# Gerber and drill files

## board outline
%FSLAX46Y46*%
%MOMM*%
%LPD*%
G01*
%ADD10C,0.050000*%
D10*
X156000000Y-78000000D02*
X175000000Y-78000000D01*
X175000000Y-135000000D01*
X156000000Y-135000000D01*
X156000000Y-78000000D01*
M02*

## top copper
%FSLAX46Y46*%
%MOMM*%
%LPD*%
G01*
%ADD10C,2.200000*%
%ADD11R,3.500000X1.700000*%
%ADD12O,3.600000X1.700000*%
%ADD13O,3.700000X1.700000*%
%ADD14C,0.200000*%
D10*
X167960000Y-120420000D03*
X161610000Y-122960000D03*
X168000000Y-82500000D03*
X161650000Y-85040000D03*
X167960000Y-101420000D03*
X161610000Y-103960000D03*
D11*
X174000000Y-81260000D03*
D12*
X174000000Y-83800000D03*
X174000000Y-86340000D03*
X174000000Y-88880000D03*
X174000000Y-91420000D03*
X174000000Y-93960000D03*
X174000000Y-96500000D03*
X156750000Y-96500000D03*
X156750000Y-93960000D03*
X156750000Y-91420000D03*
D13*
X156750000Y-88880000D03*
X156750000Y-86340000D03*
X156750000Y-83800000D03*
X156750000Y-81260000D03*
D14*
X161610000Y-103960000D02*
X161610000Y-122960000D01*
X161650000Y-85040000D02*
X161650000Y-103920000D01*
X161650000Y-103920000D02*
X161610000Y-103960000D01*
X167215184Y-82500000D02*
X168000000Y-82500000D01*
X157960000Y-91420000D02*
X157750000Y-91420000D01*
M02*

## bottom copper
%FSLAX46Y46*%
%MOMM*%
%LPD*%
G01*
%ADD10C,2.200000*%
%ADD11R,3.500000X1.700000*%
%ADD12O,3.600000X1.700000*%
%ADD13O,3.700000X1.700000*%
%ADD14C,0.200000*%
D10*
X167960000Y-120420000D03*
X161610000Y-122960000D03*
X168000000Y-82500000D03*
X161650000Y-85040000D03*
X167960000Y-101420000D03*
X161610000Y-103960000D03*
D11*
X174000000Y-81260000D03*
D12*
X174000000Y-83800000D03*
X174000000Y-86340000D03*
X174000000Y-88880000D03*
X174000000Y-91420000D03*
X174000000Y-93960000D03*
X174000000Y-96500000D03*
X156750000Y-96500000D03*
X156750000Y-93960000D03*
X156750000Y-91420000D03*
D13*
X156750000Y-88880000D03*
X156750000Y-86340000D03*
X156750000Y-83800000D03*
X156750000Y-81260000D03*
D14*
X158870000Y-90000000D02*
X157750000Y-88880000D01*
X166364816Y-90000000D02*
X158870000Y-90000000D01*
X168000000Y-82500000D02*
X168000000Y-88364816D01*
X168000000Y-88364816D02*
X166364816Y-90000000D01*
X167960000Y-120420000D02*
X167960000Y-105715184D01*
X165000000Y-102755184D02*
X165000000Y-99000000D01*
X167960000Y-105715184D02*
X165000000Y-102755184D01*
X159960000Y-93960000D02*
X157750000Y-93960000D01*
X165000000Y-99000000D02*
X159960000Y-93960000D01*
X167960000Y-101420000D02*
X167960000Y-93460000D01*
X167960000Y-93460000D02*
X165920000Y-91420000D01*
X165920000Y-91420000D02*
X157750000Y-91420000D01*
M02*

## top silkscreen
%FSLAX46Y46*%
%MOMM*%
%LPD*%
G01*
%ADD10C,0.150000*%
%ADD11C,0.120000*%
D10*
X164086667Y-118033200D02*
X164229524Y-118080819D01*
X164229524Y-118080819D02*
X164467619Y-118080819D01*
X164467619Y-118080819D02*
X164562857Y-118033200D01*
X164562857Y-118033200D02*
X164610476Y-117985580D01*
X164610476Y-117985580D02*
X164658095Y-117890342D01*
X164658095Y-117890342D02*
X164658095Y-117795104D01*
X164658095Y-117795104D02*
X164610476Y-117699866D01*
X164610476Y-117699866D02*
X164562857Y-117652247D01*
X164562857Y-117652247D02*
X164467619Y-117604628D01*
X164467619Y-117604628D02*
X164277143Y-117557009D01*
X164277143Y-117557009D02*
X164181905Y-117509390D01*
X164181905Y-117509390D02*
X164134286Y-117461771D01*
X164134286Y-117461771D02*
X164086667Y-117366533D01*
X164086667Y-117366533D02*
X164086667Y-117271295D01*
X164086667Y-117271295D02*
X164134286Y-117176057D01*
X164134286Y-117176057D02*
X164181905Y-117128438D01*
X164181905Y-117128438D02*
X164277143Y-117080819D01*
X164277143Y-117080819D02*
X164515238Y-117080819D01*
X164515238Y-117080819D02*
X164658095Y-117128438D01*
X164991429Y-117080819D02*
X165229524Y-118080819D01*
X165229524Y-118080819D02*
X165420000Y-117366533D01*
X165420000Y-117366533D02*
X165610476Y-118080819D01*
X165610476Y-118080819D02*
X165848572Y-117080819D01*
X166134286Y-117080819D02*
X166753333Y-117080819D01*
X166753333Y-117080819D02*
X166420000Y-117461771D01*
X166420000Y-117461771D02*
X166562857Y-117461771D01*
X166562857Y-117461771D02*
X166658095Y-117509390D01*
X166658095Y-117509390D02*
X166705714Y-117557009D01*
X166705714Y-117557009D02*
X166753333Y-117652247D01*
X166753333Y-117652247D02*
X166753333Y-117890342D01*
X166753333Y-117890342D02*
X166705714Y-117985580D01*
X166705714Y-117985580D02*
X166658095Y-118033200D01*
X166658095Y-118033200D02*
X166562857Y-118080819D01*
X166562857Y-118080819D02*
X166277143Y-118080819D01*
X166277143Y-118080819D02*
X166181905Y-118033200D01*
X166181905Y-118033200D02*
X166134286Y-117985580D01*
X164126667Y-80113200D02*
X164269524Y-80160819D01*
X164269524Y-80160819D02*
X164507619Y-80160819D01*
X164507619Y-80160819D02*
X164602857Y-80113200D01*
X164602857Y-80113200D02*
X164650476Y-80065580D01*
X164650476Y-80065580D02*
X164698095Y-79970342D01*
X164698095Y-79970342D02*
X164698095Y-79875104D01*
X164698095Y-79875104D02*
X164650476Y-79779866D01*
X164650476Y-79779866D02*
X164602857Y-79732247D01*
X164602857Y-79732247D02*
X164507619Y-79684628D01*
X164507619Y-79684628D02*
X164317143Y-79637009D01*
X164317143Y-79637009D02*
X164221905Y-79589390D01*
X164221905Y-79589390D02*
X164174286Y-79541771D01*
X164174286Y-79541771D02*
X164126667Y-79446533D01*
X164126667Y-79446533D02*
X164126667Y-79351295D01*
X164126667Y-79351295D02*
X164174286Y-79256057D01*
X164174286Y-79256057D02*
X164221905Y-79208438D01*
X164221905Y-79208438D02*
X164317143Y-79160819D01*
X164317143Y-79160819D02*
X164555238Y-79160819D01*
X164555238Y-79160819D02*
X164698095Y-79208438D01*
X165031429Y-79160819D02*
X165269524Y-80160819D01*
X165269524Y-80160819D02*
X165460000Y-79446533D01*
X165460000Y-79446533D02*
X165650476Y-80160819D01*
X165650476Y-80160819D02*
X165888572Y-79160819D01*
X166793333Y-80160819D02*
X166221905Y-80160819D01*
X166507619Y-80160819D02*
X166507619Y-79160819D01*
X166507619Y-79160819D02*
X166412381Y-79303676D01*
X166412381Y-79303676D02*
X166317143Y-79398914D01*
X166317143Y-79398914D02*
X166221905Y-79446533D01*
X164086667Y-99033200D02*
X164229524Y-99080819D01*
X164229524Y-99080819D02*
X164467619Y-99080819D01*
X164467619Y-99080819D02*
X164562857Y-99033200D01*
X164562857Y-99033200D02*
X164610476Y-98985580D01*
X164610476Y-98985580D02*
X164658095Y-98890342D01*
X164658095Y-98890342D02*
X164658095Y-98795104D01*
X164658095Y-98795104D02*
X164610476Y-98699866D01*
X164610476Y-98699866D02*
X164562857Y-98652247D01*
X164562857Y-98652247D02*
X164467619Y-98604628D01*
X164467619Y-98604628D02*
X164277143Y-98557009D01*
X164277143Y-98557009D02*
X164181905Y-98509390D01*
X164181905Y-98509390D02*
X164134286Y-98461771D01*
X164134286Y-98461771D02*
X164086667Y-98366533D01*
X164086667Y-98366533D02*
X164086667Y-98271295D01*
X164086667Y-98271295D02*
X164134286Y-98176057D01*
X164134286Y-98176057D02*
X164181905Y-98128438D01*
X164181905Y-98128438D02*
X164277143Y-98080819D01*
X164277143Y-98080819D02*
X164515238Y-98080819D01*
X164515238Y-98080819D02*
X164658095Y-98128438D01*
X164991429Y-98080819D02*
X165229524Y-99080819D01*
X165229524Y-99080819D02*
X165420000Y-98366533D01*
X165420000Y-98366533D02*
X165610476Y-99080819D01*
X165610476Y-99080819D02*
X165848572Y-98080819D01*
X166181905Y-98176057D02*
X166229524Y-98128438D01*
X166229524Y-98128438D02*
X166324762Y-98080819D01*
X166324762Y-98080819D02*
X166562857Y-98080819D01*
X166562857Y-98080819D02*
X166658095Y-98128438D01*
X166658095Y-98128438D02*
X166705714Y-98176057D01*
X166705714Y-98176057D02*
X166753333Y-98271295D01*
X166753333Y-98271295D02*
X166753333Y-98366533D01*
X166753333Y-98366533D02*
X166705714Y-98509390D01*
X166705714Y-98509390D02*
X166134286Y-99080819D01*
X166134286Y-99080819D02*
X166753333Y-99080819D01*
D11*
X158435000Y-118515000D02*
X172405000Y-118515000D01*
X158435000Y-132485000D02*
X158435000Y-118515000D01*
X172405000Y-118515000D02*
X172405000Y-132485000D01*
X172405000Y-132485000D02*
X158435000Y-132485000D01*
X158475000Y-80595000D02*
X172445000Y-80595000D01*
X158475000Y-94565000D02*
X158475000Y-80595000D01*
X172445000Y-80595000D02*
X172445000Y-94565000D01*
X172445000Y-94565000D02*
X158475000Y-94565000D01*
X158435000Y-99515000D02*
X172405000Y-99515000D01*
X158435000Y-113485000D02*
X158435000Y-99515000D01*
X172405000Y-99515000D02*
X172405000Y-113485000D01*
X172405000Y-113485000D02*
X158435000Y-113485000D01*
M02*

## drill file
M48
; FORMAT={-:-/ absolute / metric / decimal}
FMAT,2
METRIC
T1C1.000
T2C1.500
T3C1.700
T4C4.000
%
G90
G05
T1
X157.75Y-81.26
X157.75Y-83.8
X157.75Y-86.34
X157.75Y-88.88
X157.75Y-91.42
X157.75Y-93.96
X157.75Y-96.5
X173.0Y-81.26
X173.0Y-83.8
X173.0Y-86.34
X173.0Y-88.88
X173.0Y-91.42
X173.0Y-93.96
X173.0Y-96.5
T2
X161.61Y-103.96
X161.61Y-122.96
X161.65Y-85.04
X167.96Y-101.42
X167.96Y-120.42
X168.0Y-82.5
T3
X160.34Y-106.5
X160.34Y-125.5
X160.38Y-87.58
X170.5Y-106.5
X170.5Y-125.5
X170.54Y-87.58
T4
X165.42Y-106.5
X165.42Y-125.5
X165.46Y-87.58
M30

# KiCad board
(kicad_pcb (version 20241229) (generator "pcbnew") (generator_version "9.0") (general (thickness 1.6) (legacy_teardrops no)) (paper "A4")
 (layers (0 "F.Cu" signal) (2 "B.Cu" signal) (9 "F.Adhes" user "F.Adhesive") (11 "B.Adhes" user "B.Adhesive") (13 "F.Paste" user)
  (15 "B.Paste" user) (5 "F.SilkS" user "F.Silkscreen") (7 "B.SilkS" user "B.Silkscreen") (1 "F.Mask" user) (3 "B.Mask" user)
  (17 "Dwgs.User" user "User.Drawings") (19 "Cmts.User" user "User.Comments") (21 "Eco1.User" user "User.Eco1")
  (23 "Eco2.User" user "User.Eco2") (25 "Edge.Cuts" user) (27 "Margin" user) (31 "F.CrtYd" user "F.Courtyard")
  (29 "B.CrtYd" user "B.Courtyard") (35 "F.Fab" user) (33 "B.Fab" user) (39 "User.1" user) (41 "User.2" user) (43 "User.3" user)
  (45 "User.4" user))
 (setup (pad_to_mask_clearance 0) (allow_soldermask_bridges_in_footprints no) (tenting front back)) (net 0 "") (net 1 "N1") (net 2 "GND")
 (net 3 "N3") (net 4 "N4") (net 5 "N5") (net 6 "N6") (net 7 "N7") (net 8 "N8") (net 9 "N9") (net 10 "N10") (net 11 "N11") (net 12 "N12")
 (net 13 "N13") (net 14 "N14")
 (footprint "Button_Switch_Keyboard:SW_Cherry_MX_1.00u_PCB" (layer "F.Cu") (at 167.96 120.42)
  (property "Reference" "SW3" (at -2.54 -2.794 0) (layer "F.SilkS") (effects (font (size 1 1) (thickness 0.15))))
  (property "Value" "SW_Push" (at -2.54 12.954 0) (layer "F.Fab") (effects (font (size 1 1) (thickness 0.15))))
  (fp_line (start -9.525 -1.905) (end 4.445 -1.905) (stroke (width 0.12) (type solid)) (layer "F.SilkS"))
  (fp_line (start -9.525 12.065) (end -9.525 -1.905) (stroke (width 0.12) (type solid)) (layer "F.SilkS"))
  (fp_line (start 4.445 -1.905) (end 4.445 12.065) (stroke (width 0.12) (type solid)) (layer "F.SilkS"))
  (fp_line (start 4.445 12.065) (end -9.525 12.065) (stroke (width 0.12) (type solid)) (layer "F.SilkS"))
  (pad "" np_thru_hole circle (at -7.62 5.08) (size 1.7 1.7) (drill 1.7) (layers "*.Cu" "*.Mask"))
  (pad "" np_thru_hole circle (at -2.54 5.08) (size 4 4) (drill 4) (layers "*.Cu" "*.Mask"))
  (pad "" np_thru_hole circle (at 2.54 5.08) (size 1.7 1.7) (drill 1.7) (layers "*.Cu" "*.Mask"))
  (pad "1" thru_hole circle (at 0 0) (size 2.2 2.2) (drill 1.5) (layers "*.Cu" "*.Mask") (remove_unused_layers no) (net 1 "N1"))
  (pad "2" thru_hole circle (at -6.35 2.54) (size 2.2 2.2) (drill 1.5) (layers "*.Cu" "*.Mask") (remove_unused_layers no) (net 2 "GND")))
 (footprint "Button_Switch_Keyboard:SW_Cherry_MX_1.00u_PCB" (layer "F.Cu") (at 168 82.5)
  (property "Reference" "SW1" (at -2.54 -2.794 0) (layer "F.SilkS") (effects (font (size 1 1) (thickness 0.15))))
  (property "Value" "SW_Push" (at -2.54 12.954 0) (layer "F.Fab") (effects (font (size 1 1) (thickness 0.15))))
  (fp_line (start -9.525 -1.905) (end 4.445 -1.905) (stroke (width 0.12) (type solid)) (layer "F.SilkS"))
  (fp_line (start -9.525 12.065) (end -9.525 -1.905) (stroke (width 0.12) (type solid)) (layer "F.SilkS"))
  (fp_line (start 4.445 -1.905) (end 4.445 12.065) (stroke (width 0.12) (type solid)) (layer "F.SilkS"))
  (fp_line (start 4.445 12.065) (end -9.525 12.065) (stroke (width 0.12) (type solid)) (layer "F.SilkS"))
  (pad "" np_thru_hole circle (at -7.62 5.08) (size 1.7 1.7) (drill 1.7) (layers "*.Cu" "*.Mask"))
  (pad "" np_thru_hole circle (at -2.54 5.08) (size 4 4) (drill 4) (layers "*.Cu" "*.Mask"))
  (pad "" np_thru_hole circle (at 2.54 5.08) (size 1.7 1.7) (drill 1.7) (layers "*.Cu" "*.Mask"))
  (pad "1" thru_hole circle (at 0 0) (size 2.2 2.2) (drill 1.5) (layers "*.Cu" "*.Mask") (remove_unused_layers no) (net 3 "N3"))
  (pad "2" thru_hole circle (at -6.35 2.54) (size 2.2 2.2) (drill 1.5) (layers "*.Cu" "*.Mask") (remove_unused_layers no) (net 2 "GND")))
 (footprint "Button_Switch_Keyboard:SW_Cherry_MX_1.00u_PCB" (layer "F.Cu") (at 167.96 101.42)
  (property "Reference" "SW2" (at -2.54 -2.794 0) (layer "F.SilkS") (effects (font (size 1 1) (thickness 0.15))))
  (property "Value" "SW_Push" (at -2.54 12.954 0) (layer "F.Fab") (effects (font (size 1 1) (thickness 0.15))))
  (fp_line (start -9.525 -1.905) (end 4.445 -1.905) (stroke (width 0.12) (type solid)) (layer "F.SilkS"))
  (fp_line (start -9.525 12.065) (end -9.525 -1.905) (stroke (width 0.12) (type solid)) (layer "F.SilkS"))
  (fp_line (start 4.445 -1.905) (end 4.445 12.065) (stroke (width 0.12) (type solid)) (layer "F.SilkS"))
  (fp_line (start 4.445 12.065) (end -9.525 12.065) (stroke (width 0.12) (type solid)) (layer "F.SilkS"))
  (pad "" np_thru_hole circle (at -7.62 5.08) (size 1.7 1.7) (drill 1.7) (layers "*.Cu" "*.Mask"))
  (pad "" np_thru_hole circle (at -2.54 5.08) (size 4 4) (drill 4) (layers "*.Cu" "*.Mask"))
  (pad "" np_thru_hole circle (at 2.54 5.08) (size 1.7 1.7) (drill 1.7) (layers "*.Cu" "*.Mask"))
  (pad "1" thru_hole circle (at 0 0) (size 2.2 2.2) (drill 1.5) (layers "*.Cu" "*.Mask") (remove_unused_layers no) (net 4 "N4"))
  (pad "2" thru_hole circle (at -6.35 2.54) (size 2.2 2.2) (drill 1.5) (layers "*.Cu" "*.Mask") (remove_unused_layers no) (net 2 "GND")))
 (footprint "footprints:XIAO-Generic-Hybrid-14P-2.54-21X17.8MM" (layer "B.Cu") (at 165.375 88.88 180)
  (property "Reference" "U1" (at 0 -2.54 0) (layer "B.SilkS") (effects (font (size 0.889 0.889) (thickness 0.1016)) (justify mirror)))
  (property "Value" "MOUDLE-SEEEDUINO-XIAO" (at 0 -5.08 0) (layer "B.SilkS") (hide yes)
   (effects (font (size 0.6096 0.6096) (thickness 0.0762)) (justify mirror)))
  (pad "1" thru_hole rect (at -7.625 7.62 180) (size 3.5 1.7) (drill 1 (offset -1 0)) (layers "*.Cu" "*.Mask") (remove_unused_layers no)
   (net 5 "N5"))
  (pad "2" thru_hole oval (at -7.625 5.08 180) (size 3.6 1.7) (drill 1 (offset -1 0)) (layers "*.Cu" "*.Mask") (remove_unused_layers no)
   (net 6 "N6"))
  (pad "3" thru_hole oval (at -7.625 2.54 180) (size 3.6 1.7) (drill 1 (offset -1 0)) (layers "*.Cu" "*.Mask") (remove_unused_layers no)
   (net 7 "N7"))
  (pad "4" thru_hole oval (at -7.625 0 180) (size 3.6 1.7) (drill 1 (offset -1 0)) (layers "*.Cu" "*.Mask") (remove_unused_layers no)
   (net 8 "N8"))
  (pad "5" thru_hole oval (at -7.625 -2.54 180) (size 3.6 1.7) (drill 1 (offset -1 0)) (layers "*.Cu" "*.Mask") (remove_unused_layers no)
   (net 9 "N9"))
  (pad "6" thru_hole oval (at -7.625 -5.08) (size 3.6 1.7) (drill 1 (offset 1 0)) (layers "*.Cu" "*.Mask") (remove_unused_layers no)
   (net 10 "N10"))
  (pad "7" thru_hole oval (at -7.625 -7.62 180) (size 3.6 1.7) (drill 1 (offset -1 0)) (layers "*.Cu" "*.Mask") (remove_unused_layers no)
   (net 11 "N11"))
  (pad "8" thru_hole oval (at 7.625 -7.62 180) (size 3.6 1.7) (drill 1 (offset 1 0)) (layers "*.Cu" "*.Mask") (remove_unused_layers no)
   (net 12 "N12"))
  (pad "9" thru_hole oval (at 7.625 -5.08 180) (size 3.6 1.7) (drill 1 (offset 1 0)) (layers "*.Cu" "*.Mask") (remove_unused_layers no)
   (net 1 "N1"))
  (pad "10" thru_hole oval (at 7.625 -2.54 180) (size 3.6 1.7) (drill 1 (offset 1 0)) (layers "*.Cu" "*.Mask") (remove_unused_layers no)
   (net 4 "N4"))
  (pad "11" thru_hole oval (at 7.625 0 180) (size 3.7 1.7) (drill 1 (offset 1 0)) (layers "*.Cu" "*.Mask") (remove_unused_layers no)
   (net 3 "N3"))
  (pad "12" thru_hole oval (at 7.625 2.54 180) (size 3.7 1.7) (drill 1 (offset 1 0)) (layers "*.Cu" "*.Mask") (remove_unused_layers no)
   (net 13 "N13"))
  (pad "13" thru_hole oval (at 7.625 5.08 180) (size 3.7 1.7) (drill 1 (offset 1 0)) (layers "*.Cu" "*.Mask") (remove_unused_layers no)
   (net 2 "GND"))
  (pad "14" thru_hole oval (at 7.625 7.62 180) (size 3.7 1.7) (drill 1 (offset 1 0)) (layers "*.Cu" "*.Mask") (remove_unused_layers no)
   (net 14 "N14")))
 (gr_rect (start 156 78) (end 175 135) (stroke (width 0.05) (type default)) (fill no) (layer "Edge.Cuts"))
 (segment (start 161.61 103.96) (end 161.61 122.96) (width 0.2) (layer "F.Cu") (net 2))
 (segment (start 161.65 85.04) (end 161.65 103.92) (width 0.2) (layer "F.Cu") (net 2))
 (segment (start 161.65 103.92) (end 161.61 103.96) (width 0.2) (layer "F.Cu") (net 2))
 (segment (start 167.215184 82.5) (end 168 82.5) (width 0.2) (layer "F.Cu") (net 3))
 (segment (start 158.87 90) (end 157.75 88.88) (width 0.2) (layer "B.Cu") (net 3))
 (segment (start 166.364816 90) (end 158.87 90) (width 0.2) (layer "B.Cu") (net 3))
 (segment (start 168 82.5) (end 168 88.364816) (width 0.2) (layer "B.Cu") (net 3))
 (segment (start 168 88.364816) (end 166.364816 90) (width 0.2) (layer "B.Cu") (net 3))
 (segment (start 167.96 120.42) (end 167.96 105.715184) (width 0.2) (layer "B.Cu") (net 1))
 (segment (start 165 102.755184) (end 165 99) (width 0.2) (layer "B.Cu") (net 1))
 (segment (start 167.96 105.715184) (end 165 102.755184) (width 0.2) (layer "B.Cu") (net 1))
 (segment (start 159.96 93.96) (end 157.75 93.96) (width 0.2) (layer "B.Cu") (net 1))
 (segment (start 165 99) (end 159.96 93.96) (width 0.2) (layer "B.Cu") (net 1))
 (segment (start 157.96 91.42) (end 157.75 91.42) (width 0.2) (layer "F.Cu") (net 4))
 (segment (start 167.96 101.42) (end 167.96 93.46) (width 0.2) (layer "B.Cu") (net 4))
 (segment (start 167.96 93.46) (end 165.92 91.42) (width 0.2) (layer "B.Cu") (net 4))
 (segment (start 165.92 91.42) (end 157.75 91.42) (width 0.2) (layer "B.Cu") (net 4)))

